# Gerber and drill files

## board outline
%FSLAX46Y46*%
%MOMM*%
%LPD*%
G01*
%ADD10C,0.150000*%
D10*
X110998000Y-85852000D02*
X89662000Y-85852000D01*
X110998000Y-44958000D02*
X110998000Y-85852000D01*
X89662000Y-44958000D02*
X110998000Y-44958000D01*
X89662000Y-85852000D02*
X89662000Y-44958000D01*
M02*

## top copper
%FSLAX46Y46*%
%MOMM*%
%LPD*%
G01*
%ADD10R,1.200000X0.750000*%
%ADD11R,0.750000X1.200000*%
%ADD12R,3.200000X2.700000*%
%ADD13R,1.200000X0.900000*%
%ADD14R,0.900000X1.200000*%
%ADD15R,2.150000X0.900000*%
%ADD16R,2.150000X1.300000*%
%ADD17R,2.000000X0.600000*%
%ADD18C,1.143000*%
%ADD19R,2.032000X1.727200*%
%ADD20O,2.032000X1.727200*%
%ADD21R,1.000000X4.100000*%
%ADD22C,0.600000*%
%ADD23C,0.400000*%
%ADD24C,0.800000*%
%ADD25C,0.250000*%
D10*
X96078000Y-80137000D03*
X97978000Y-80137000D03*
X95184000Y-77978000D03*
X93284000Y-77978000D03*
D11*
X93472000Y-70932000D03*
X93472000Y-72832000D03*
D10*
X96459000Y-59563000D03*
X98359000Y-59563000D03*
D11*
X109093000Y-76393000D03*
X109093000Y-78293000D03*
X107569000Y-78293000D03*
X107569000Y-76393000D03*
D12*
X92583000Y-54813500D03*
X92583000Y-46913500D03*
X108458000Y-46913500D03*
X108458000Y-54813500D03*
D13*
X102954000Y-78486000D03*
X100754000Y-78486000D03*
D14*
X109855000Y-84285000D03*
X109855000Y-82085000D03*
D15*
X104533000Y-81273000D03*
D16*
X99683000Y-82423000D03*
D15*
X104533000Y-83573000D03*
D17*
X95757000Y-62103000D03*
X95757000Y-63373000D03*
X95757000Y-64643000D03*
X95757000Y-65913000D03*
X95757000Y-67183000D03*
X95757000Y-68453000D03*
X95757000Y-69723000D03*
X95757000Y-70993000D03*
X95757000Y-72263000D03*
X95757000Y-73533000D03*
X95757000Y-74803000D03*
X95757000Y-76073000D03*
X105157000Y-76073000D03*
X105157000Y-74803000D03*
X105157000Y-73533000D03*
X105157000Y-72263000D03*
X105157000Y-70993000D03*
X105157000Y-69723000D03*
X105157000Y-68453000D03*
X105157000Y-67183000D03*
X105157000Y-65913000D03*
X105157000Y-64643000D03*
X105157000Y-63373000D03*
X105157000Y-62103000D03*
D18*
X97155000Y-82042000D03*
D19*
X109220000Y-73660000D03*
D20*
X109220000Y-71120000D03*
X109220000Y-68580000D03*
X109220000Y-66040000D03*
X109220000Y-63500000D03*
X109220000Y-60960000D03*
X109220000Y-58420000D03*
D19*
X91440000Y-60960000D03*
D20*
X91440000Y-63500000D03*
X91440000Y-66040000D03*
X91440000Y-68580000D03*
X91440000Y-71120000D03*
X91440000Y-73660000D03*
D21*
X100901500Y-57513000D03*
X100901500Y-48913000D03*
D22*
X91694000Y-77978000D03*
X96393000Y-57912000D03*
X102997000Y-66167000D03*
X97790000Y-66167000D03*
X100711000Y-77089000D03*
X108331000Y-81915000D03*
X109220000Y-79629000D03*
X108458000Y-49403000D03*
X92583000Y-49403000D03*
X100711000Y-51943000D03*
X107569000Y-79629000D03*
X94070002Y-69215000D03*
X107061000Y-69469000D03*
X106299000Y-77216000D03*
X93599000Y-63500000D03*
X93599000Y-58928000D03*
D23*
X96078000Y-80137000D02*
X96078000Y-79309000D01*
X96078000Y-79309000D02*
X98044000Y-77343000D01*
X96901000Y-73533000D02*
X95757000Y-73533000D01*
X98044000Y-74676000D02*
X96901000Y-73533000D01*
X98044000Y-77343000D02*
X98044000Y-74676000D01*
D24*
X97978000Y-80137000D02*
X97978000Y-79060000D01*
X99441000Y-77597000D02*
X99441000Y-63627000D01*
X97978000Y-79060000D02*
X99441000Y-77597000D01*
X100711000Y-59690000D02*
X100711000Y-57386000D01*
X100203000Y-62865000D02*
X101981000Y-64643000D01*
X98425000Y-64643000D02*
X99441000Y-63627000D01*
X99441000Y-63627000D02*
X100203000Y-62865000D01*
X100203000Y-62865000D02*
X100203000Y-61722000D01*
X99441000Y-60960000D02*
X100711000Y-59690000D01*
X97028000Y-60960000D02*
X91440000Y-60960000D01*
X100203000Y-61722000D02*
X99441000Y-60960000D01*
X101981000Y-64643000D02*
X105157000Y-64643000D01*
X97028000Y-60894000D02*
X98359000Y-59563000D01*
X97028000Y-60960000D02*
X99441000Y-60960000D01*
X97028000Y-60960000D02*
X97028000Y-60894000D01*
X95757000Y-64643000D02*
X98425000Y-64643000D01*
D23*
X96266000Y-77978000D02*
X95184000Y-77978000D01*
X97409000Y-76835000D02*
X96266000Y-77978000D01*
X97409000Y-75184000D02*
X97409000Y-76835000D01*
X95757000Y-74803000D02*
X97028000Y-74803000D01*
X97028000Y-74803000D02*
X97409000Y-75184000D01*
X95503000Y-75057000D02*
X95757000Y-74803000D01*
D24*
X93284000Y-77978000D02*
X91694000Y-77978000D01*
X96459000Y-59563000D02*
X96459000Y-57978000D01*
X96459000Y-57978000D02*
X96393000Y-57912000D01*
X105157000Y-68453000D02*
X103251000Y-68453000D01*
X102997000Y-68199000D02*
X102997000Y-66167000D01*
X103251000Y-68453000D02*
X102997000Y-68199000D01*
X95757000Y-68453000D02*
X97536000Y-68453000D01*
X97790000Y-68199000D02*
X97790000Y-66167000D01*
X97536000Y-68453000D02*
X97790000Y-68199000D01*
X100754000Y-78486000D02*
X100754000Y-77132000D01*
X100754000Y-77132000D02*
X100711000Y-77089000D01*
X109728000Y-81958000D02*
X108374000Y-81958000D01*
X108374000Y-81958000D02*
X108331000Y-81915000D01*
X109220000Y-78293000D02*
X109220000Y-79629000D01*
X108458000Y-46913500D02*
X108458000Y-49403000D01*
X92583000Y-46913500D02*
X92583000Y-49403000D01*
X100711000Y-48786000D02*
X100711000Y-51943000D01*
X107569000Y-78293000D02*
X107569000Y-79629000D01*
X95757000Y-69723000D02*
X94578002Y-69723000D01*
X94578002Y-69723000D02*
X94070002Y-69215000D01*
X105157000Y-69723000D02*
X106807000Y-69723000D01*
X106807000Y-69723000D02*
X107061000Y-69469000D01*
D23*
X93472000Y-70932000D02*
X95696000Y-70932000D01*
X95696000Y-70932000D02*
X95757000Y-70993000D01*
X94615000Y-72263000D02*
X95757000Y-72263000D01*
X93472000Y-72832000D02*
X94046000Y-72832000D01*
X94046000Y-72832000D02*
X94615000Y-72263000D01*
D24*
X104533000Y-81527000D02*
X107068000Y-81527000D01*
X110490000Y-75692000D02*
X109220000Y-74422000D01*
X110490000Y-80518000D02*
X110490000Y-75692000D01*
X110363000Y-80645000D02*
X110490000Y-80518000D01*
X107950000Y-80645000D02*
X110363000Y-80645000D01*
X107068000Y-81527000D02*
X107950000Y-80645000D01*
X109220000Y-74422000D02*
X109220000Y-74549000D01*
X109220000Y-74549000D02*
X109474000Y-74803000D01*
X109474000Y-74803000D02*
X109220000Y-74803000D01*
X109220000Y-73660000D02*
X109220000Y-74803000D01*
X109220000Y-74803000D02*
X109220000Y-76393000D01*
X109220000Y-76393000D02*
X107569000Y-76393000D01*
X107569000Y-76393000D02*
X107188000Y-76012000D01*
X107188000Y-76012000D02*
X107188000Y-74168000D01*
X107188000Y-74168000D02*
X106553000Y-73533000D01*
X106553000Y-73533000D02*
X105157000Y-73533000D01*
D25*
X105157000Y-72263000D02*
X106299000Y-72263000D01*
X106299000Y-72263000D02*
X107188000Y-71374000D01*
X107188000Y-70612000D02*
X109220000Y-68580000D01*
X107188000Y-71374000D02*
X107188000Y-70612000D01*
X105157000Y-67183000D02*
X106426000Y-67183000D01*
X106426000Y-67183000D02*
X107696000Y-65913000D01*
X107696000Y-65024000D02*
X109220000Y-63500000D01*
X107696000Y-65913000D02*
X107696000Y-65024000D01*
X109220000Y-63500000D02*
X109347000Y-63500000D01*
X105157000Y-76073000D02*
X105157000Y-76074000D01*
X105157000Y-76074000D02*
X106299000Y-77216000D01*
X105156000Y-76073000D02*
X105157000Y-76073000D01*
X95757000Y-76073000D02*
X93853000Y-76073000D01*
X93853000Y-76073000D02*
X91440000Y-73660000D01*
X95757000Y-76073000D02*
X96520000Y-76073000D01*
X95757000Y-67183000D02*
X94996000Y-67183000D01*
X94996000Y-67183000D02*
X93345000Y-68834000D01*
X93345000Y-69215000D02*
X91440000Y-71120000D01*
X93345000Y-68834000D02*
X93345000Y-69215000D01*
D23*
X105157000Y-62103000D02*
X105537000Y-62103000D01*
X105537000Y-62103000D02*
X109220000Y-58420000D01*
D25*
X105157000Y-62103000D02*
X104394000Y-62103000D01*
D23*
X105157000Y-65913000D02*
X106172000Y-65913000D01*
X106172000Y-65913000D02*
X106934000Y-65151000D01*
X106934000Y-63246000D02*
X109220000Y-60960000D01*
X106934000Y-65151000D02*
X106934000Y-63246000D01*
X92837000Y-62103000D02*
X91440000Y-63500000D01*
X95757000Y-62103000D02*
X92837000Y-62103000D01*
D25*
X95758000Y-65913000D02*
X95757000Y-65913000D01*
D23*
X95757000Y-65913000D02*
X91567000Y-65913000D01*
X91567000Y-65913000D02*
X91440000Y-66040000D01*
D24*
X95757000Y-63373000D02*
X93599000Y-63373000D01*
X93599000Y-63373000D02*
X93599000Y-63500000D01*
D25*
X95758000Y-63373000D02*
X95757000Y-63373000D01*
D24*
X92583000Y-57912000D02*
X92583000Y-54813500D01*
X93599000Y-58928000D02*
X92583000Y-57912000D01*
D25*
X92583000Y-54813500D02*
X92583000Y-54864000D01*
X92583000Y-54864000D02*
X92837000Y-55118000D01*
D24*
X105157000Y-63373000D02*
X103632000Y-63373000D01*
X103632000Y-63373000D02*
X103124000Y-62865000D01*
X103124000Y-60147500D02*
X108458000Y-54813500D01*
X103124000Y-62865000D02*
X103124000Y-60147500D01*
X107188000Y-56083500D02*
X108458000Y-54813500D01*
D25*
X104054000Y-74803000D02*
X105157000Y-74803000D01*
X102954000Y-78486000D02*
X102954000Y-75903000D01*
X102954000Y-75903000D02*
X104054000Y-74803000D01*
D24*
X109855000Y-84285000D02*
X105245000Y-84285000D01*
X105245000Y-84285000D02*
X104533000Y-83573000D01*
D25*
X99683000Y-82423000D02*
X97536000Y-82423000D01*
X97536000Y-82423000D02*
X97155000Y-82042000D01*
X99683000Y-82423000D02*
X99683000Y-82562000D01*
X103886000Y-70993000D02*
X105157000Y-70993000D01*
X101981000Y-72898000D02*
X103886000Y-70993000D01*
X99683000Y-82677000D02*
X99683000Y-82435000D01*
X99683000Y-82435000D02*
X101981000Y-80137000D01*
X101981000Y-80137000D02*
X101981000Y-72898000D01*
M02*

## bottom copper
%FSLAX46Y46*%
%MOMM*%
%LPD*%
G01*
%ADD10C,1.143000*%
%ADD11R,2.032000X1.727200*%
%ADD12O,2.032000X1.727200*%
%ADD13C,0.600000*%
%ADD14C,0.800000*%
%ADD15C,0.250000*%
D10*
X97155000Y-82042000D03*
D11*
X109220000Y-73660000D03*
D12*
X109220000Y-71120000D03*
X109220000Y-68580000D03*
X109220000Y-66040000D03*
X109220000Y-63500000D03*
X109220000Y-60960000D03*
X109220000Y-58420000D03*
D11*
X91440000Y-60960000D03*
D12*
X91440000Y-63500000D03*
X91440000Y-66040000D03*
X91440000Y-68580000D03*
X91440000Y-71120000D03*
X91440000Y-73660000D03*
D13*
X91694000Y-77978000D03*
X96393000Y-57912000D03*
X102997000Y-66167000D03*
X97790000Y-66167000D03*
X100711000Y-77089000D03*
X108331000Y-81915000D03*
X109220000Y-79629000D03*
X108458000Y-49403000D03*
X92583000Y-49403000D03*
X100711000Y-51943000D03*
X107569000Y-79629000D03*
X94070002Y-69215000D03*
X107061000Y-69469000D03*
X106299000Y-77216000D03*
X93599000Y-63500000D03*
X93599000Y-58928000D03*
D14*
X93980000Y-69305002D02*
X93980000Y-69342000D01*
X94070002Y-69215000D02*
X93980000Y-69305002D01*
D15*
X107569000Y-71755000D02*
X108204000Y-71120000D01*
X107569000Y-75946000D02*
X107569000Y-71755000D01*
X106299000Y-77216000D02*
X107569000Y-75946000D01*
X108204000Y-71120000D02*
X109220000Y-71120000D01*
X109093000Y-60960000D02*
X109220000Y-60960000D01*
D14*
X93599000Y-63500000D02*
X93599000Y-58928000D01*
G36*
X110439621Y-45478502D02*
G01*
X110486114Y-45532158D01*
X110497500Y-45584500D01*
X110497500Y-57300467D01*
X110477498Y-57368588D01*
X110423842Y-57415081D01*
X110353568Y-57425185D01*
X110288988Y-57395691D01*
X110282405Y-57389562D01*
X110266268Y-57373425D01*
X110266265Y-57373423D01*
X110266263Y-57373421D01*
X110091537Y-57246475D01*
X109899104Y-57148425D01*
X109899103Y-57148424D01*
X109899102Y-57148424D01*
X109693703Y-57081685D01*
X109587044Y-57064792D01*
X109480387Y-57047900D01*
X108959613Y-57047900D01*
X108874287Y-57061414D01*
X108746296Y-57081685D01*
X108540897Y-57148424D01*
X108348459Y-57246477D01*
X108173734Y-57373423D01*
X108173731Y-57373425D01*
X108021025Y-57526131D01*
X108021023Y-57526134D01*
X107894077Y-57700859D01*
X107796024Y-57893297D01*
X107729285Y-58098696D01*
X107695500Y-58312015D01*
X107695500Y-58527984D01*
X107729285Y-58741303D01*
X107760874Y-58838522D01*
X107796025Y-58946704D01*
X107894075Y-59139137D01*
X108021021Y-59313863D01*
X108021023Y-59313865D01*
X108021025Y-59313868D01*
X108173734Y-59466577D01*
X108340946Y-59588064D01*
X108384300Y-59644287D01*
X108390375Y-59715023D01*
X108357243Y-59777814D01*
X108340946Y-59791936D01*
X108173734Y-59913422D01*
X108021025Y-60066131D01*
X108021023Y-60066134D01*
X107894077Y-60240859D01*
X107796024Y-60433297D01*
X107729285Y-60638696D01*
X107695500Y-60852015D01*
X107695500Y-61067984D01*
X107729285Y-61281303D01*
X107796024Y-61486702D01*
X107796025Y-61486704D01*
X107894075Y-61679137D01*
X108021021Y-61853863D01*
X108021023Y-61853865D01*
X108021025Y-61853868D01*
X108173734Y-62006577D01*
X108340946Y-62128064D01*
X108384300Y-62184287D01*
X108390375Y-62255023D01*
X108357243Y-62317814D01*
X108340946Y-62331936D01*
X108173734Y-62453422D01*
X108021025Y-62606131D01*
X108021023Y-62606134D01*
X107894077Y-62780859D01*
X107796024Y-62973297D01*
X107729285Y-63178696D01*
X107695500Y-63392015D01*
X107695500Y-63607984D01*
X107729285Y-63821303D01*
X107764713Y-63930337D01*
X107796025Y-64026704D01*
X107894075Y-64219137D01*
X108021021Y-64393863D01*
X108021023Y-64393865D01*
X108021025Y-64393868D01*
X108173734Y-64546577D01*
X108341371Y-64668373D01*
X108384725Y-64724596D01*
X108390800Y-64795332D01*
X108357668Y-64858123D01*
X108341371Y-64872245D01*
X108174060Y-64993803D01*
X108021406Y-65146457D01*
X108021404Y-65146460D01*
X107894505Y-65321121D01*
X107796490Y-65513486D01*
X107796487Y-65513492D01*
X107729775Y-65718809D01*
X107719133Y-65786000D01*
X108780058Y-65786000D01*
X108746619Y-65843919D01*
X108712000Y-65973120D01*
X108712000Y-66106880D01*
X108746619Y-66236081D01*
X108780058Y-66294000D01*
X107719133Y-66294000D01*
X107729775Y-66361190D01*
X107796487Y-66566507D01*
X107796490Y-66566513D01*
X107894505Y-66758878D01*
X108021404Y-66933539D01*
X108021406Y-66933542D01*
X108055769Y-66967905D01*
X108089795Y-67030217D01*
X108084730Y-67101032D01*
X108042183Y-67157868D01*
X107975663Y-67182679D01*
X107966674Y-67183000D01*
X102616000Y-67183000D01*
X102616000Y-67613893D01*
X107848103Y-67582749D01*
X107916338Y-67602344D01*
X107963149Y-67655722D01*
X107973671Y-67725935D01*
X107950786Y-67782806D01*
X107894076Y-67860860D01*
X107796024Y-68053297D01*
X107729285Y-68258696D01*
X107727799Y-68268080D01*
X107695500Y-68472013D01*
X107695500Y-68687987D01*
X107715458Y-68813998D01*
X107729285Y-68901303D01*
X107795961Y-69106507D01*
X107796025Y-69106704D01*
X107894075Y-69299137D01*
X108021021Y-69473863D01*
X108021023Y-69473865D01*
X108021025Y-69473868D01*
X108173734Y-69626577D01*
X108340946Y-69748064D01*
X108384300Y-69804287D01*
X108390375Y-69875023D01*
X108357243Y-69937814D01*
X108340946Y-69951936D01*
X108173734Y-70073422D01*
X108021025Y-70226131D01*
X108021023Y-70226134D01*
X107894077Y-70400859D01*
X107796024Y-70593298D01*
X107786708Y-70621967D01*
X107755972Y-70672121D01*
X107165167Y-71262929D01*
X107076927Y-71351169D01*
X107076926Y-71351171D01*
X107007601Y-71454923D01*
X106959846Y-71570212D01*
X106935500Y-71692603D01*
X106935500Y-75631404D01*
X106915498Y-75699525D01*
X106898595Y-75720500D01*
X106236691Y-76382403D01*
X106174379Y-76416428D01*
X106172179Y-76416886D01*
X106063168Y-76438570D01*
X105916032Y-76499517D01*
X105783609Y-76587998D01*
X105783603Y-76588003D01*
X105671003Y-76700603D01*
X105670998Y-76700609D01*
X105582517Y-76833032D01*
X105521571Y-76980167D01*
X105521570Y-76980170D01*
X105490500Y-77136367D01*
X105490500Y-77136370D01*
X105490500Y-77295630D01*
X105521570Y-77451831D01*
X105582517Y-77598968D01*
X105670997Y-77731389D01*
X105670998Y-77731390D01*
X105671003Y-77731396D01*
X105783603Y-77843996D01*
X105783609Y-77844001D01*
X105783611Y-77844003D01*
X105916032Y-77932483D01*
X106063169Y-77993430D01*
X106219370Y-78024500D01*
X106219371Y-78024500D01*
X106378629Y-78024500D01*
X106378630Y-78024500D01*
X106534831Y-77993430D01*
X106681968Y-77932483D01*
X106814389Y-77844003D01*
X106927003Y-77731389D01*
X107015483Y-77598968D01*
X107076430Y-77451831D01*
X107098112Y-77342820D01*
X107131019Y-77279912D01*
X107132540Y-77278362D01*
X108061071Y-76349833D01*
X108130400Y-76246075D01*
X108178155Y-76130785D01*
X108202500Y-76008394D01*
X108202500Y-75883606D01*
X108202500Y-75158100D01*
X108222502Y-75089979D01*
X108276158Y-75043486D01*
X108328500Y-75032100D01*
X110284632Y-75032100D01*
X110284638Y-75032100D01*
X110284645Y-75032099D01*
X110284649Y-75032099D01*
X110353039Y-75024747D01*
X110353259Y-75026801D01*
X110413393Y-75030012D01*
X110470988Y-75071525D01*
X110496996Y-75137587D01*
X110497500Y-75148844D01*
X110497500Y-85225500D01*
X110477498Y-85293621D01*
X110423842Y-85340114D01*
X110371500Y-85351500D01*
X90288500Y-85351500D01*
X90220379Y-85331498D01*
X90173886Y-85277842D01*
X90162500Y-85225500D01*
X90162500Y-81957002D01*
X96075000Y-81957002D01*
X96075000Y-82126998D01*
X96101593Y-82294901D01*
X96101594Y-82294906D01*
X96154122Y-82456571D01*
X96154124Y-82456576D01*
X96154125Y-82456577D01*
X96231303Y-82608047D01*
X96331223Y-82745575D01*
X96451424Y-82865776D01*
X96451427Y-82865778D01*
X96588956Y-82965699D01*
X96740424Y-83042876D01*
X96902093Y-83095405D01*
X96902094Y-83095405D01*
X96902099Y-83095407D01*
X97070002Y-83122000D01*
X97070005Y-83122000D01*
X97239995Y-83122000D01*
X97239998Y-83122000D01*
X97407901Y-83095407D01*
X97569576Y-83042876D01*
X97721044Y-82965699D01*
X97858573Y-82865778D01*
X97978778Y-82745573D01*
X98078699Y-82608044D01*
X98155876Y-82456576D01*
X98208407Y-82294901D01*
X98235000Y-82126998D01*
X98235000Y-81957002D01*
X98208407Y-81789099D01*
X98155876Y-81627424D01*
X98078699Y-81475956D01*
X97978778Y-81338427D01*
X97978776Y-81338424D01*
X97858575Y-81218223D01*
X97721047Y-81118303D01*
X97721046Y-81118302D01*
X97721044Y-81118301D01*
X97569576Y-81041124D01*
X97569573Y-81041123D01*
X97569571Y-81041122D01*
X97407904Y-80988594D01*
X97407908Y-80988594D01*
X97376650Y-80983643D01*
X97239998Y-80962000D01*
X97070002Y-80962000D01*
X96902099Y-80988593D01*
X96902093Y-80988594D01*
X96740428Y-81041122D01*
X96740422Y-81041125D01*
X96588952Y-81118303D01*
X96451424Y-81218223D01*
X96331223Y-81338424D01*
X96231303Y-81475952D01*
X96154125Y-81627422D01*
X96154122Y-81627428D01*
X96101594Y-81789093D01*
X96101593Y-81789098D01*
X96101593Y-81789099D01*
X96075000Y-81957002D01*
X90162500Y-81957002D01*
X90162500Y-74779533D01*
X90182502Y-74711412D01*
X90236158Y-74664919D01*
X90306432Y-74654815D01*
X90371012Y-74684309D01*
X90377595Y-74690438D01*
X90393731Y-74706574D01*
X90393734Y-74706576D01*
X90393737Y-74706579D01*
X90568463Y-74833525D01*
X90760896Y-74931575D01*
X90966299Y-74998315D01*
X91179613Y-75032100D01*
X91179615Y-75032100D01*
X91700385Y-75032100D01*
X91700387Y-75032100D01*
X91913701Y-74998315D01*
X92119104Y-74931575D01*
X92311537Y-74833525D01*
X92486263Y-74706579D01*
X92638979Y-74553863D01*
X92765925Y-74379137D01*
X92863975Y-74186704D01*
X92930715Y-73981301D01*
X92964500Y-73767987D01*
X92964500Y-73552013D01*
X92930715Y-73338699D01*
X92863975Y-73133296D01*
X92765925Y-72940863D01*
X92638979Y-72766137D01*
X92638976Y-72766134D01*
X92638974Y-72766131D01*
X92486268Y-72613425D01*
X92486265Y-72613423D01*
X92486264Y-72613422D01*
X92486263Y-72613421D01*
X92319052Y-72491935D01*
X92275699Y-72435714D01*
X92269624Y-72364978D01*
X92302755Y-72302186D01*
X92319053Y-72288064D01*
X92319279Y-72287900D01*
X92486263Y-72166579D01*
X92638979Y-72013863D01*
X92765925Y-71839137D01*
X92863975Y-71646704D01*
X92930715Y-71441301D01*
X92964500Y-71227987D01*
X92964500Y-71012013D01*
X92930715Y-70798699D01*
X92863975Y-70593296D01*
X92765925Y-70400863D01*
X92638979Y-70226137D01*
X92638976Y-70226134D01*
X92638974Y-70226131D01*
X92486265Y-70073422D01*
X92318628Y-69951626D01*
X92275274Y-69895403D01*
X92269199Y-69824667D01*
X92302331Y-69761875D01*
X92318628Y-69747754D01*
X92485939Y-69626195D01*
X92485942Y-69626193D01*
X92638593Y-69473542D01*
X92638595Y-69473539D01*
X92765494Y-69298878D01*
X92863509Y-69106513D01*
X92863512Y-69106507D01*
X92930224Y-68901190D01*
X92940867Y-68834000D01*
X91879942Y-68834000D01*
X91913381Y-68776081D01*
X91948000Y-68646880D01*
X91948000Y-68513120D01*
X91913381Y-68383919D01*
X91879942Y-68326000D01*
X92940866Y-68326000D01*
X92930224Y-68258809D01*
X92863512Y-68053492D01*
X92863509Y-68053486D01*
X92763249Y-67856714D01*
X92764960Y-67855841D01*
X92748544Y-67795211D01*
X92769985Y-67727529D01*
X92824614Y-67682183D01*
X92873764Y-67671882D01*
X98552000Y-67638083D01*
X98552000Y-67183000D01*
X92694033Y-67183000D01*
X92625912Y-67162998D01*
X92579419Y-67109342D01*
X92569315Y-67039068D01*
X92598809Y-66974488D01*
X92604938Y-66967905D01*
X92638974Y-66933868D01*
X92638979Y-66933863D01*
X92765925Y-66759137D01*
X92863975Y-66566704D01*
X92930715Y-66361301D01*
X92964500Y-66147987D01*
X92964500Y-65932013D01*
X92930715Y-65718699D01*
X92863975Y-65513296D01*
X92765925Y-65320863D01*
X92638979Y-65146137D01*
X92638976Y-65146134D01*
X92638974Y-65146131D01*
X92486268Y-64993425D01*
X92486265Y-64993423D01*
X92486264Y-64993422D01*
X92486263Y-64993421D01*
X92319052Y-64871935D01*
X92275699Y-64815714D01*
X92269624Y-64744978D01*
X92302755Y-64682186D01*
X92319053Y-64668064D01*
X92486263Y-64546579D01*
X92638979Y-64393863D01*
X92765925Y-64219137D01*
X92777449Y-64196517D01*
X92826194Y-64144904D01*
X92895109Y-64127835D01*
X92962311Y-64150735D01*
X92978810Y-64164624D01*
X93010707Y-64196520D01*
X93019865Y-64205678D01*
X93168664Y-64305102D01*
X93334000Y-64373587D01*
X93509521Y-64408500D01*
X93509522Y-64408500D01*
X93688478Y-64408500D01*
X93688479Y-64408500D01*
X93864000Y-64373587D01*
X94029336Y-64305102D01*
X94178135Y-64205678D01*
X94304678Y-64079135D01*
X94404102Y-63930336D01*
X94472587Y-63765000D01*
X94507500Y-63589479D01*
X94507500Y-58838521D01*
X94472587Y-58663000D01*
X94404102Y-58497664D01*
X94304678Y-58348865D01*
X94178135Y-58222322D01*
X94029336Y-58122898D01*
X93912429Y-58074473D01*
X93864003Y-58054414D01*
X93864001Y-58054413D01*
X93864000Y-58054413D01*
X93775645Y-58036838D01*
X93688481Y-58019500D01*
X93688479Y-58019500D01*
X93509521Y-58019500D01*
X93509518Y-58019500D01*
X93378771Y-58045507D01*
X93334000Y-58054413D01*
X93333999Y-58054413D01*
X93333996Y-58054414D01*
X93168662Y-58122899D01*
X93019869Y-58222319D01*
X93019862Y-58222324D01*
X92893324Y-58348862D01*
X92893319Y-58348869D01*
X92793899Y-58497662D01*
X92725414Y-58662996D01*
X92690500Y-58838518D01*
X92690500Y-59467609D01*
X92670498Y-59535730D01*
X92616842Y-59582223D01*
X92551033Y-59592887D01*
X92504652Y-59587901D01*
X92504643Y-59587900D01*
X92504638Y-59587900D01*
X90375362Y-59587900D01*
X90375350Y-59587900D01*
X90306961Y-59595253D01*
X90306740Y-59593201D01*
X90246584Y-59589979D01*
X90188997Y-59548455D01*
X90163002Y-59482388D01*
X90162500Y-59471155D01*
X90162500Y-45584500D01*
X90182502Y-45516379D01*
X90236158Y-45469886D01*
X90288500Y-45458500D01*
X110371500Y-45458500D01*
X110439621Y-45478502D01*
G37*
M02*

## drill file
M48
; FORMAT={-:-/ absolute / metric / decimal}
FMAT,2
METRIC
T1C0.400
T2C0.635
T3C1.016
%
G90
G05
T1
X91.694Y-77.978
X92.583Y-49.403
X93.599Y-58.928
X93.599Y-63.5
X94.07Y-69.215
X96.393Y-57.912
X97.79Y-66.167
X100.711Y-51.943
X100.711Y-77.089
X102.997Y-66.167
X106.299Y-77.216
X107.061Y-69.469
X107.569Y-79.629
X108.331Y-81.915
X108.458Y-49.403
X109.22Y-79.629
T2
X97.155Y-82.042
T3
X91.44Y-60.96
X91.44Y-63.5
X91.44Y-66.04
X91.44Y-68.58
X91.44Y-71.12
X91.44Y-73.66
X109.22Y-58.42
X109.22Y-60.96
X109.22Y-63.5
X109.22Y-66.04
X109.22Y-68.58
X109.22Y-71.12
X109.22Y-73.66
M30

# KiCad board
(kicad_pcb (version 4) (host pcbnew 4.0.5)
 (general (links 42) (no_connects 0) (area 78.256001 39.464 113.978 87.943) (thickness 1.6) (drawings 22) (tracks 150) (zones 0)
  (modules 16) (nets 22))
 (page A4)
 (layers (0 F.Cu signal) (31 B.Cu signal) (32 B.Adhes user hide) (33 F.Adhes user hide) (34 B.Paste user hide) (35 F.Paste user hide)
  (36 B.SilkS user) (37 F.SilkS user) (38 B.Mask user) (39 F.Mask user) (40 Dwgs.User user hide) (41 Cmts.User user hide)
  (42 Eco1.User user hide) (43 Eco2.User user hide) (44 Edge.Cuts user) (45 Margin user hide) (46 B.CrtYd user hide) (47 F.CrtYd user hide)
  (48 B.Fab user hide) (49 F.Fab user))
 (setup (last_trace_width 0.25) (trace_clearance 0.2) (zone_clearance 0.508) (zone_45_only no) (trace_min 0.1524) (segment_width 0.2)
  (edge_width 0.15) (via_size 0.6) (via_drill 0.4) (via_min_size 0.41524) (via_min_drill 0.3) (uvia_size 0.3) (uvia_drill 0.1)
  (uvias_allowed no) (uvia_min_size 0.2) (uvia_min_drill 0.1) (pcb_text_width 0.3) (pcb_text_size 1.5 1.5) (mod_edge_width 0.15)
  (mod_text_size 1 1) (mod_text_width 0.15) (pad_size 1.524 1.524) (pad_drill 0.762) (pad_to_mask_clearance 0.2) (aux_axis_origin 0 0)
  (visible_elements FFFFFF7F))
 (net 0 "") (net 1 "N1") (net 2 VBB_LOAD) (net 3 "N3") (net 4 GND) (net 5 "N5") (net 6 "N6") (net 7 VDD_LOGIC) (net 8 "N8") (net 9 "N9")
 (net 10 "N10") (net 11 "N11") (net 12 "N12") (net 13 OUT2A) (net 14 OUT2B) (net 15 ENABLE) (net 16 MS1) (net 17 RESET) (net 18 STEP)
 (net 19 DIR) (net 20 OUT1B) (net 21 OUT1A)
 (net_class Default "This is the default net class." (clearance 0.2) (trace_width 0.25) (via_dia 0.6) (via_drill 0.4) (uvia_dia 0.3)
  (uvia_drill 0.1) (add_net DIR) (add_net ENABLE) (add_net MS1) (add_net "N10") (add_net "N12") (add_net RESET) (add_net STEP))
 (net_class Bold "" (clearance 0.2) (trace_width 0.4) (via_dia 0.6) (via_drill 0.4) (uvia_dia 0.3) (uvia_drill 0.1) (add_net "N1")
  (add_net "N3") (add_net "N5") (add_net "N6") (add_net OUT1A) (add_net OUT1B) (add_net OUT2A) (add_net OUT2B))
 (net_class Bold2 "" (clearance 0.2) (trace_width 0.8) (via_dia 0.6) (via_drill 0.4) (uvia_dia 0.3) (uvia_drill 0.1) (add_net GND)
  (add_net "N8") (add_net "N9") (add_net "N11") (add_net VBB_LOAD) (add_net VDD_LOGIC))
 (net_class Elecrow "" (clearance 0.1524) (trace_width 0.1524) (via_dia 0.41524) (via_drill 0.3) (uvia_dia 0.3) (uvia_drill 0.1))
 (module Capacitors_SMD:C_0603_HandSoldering (layer F.Cu) (at 97.028 80.137)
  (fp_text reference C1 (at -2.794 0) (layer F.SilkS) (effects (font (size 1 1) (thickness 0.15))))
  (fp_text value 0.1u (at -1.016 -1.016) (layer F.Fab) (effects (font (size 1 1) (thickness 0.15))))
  (pad 1 smd rect (at -0.95 0) (size 1.2 0.75) (layers F.Cu F.Paste F.Mask) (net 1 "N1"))
  (pad 2 smd rect (at 0.95 0) (size 1.2 0.75) (layers F.Cu F.Paste F.Mask) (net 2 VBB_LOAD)))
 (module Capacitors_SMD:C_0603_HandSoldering (layer F.Cu) (at 94.234 77.978 180)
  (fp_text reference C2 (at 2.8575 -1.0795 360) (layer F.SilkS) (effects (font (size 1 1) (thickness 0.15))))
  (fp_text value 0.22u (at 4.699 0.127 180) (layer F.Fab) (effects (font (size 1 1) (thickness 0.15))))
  (pad 1 smd rect (at -0.95 0 180) (size 1.2 0.75) (layers F.Cu F.Paste F.Mask) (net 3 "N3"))
  (pad 2 smd rect (at 0.95 0 180) (size 1.2 0.75) (layers F.Cu F.Paste F.Mask) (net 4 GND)))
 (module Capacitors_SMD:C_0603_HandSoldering (layer F.Cu) (at 93.472 71.882 270)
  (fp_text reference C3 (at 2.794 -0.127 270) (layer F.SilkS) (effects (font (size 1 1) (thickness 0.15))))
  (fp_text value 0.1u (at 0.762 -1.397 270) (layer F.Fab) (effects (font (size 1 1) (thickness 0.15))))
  (pad 1 smd rect (at -0.95 0 270) (size 1.2 0.75) (layers F.Cu F.Paste F.Mask) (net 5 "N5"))
  (pad 2 smd rect (at 0.95 0 270) (size 1.2 0.75) (layers F.Cu F.Paste F.Mask) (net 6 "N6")))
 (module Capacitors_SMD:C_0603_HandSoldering (layer F.Cu) (at 97.409 59.563)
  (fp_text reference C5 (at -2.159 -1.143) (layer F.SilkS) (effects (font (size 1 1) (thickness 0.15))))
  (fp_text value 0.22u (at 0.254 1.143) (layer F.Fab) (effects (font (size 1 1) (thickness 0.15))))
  (pad 1 smd rect (at -0.95 0) (size 1.2 0.75) (layers F.Cu F.Paste F.Mask) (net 4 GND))
  (pad 2 smd rect (at 0.95 0) (size 1.2 0.75) (layers F.Cu F.Paste F.Mask) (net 2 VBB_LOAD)))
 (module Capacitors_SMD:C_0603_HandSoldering (layer F.Cu) (at 109.093 77.343 270)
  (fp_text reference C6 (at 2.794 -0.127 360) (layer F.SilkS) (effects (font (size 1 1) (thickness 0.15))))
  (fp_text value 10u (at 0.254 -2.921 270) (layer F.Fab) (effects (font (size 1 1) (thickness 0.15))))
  (pad 1 smd rect (at -0.95 0 270) (size 1.2 0.75) (layers F.Cu F.Paste F.Mask) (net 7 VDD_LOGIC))
  (pad 2 smd rect (at 0.95 0 270) (size 1.2 0.75) (layers F.Cu F.Paste F.Mask) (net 4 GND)))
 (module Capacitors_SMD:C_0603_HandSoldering (layer F.Cu) (at 107.569 77.343 90)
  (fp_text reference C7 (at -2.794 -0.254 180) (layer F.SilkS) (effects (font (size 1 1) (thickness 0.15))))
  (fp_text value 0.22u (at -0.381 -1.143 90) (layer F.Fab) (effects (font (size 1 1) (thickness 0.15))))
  (pad 1 smd rect (at -0.95 0 90) (size 1.2 0.75) (layers F.Cu F.Paste F.Mask) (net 4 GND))
  (pad 2 smd rect (at 0.95 0 90) (size 1.2 0.75) (layers F.Cu F.Paste F.Mask) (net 7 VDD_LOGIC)))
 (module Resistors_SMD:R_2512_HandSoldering (layer F.Cu) (at 92.583 50.8635 90)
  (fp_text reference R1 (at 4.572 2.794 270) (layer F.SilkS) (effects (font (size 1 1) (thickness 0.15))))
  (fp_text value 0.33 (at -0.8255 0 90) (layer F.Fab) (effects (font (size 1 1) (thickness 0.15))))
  (pad 1 smd rect (at -3.95 0 90) (size 2.7 3.2) (layers F.Cu F.Paste F.Mask) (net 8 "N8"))
  (pad 2 smd rect (at 3.95 0 90) (size 2.7 3.2) (layers F.Cu F.Paste F.Mask) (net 4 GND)))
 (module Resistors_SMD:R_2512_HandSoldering (layer F.Cu) (at 108.458 50.8635 270)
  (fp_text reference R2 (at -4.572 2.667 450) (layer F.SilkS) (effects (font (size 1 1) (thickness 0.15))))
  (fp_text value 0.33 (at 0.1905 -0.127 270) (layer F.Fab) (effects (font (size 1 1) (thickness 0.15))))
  (pad 1 smd rect (at -3.95 0 270) (size 2.7 3.2) (layers F.Cu F.Paste F.Mask) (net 4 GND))
  (pad 2 smd rect (at 3.95 0 270) (size 2.7 3.2) (layers F.Cu F.Paste F.Mask) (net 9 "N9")))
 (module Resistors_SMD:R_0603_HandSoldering (layer F.Cu) (at 101.854 78.486 180)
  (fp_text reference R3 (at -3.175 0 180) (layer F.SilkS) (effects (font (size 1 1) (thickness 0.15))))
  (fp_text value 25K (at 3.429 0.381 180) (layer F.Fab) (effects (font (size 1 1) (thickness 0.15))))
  (pad 1 smd rect (at -1.1 0 180) (size 1.2 0.9) (layers F.Cu F.Paste F.Mask) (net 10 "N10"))
  (pad 2 smd rect (at 1.1 0 180) (size 1.2 0.9) (layers F.Cu F.Paste F.Mask) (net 4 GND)))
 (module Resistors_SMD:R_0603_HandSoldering (layer F.Cu) (at 109.855 83.185 90)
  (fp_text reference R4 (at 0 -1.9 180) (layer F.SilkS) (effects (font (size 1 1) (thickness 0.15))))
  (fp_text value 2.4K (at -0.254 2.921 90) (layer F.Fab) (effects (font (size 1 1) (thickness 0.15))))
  (pad 1 smd rect (at -1.1 0 90) (size 1.2 0.9) (layers F.Cu F.Paste F.Mask) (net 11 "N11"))
  (pad 2 smd rect (at 1.1 0 90) (size 1.2 0.9) (layers F.Cu F.Paste F.Mask) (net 4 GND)))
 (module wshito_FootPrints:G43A (layer F.Cu) (at 102.108 82.423 90)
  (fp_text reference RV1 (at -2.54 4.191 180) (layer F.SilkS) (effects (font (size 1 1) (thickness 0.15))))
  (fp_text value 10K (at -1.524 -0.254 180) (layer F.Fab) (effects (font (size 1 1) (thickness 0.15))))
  (pad 1 smd rect (at 1.15 2.425 90) (size 0.9 2.15) (layers F.Cu F.Paste F.Mask) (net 7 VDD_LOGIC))
  (pad 2 smd rect (at 0 -2.425 90) (size 1.3 2.15) (layers F.Cu F.Paste F.Mask) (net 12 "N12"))
  (pad 3 smd rect (at -1.15 2.425 90) (size 0.9 2.15) (layers F.Cu F.Paste F.Mask) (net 11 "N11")))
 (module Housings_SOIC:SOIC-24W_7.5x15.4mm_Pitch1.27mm (layer F.Cu) (at 100.457 69.088)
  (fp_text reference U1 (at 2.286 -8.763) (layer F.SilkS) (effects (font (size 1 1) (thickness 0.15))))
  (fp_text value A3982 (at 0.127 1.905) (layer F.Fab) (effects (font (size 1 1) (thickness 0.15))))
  (pad 1 smd rect (at -4.7 -6.985) (size 2 0.6) (layers F.Cu F.Paste F.Mask) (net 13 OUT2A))
  (pad 2 smd rect (at -4.7 -5.715) (size 2 0.6) (layers F.Cu F.Paste F.Mask) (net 8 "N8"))
  (pad 3 smd rect (at -4.7 -4.445) (size 2 0.6) (layers F.Cu F.Paste F.Mask) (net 2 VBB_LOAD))
  (pad 4 smd rect (at -4.7 -3.175) (size 2 0.6) (layers F.Cu F.Paste F.Mask) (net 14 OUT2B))
  (pad 5 smd rect (at -4.7 -1.905) (size 2 0.6) (layers F.Cu F.Paste F.Mask) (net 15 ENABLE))
  (pad 6 smd rect (at -4.7 -0.635) (size 2 0.6) (layers F.Cu F.Paste F.Mask) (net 4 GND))
  (pad 7 smd rect (at -4.7 0.635) (size 2 0.6) (layers F.Cu F.Paste F.Mask) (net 4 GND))
  (pad 8 smd rect (at -4.7 1.905) (size 2 0.6) (layers F.Cu F.Paste F.Mask) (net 5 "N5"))
  (pad 9 smd rect (at -4.7 3.175) (size 2 0.6) (layers F.Cu F.Paste F.Mask) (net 6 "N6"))
  (pad 10 smd rect (at -4.7 4.445) (size 2 0.6) (layers F.Cu F.Paste F.Mask) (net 1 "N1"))
  (pad 11 smd rect (at -4.7 5.715) (size 2 0.6) (layers F.Cu F.Paste F.Mask) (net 3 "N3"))
  (pad 12 smd rect (at -4.7 6.985) (size 2 0.6) (layers F.Cu F.Paste F.Mask) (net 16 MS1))
  (pad 13 smd rect (at 4.7 6.985) (size 2 0.6) (layers F.Cu F.Paste F.Mask) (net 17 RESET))
  (pad 14 smd rect (at 4.7 5.715) (size 2 0.6) (layers F.Cu F.Paste F.Mask) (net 10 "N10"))
  (pad 15 smd rect (at 4.7 4.445) (size 2 0.6) (layers F.Cu F.Paste F.Mask) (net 7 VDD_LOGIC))
  (pad 16 smd rect (at 4.7 3.175) (size 2 0.6) (layers F.Cu F.Paste F.Mask) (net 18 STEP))
  (pad 17 smd rect (at 4.7 1.905) (size 2 0.6) (layers F.Cu F.Paste F.Mask) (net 12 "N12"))
  (pad 18 smd rect (at 4.7 0.635) (size 2 0.6) (layers F.Cu F.Paste F.Mask) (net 4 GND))
  (pad 19 smd rect (at 4.7 -0.635) (size 2 0.6) (layers F.Cu F.Paste F.Mask) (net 4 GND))
  (pad 20 smd rect (at 4.7 -1.905) (size 2 0.6) (layers F.Cu F.Paste F.Mask) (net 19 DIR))
  (pad 21 smd rect (at 4.7 -3.175) (size 2 0.6) (layers F.Cu F.Paste F.Mask) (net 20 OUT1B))
  (pad 22 smd rect (at 4.7 -4.445) (size 2 0.6) (layers F.Cu F.Paste F.Mask) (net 2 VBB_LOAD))
  (pad 23 smd rect (at 4.7 -5.715) (size 2 0.6) (layers F.Cu F.Paste F.Mask) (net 9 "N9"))
  (pad 24 smd rect (at 4.7 -6.985) (size 2 0.6) (layers F.Cu F.Paste F.Mask) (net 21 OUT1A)))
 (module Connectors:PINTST (layer F.Cu) (at 97.155 82.042)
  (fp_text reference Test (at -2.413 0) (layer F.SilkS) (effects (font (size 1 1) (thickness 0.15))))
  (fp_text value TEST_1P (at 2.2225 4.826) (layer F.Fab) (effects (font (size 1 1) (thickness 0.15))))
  (pad 1 thru_hole circle (at 0 0) (size 1.143 1.143) (drill 0.635) (layers *.Cu *.Mask) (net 12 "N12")))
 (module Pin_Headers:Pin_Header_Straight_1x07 (layer F.Cu) (at 109.22 73.66 180)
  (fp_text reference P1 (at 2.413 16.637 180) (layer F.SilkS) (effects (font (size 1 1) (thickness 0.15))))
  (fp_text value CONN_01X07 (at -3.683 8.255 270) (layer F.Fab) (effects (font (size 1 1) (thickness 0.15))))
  (pad 1 thru_hole rect (at 0 0 180) (size 2.032 1.7272) (drill 1.016) (layers *.Cu *.Mask) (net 7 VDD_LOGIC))
  (pad 2 thru_hole oval (at 0 2.54 180) (size 2.032 1.7272) (drill 1.016) (layers *.Cu *.Mask) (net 17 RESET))
  (pad 3 thru_hole oval (at 0 5.08 180) (size 2.032 1.7272) (drill 1.016) (layers *.Cu *.Mask) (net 18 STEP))
  (pad 4 thru_hole oval (at 0 7.62 180) (size 2.032 1.7272) (drill 1.016) (layers *.Cu *.Mask) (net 4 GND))
  (pad 5 thru_hole oval (at 0 10.16 180) (size 2.032 1.7272) (drill 1.016) (layers *.Cu *.Mask) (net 19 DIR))
  (pad 6 thru_hole oval (at 0 12.7 180) (size 2.032 1.7272) (drill 1.016) (layers *.Cu *.Mask) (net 20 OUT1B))
  (pad 7 thru_hole oval (at 0 15.24 180) (size 2.032 1.7272) (drill 1.016) (layers *.Cu *.Mask) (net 21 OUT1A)))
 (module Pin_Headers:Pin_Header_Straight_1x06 (layer F.Cu) (at 91.44 60.96)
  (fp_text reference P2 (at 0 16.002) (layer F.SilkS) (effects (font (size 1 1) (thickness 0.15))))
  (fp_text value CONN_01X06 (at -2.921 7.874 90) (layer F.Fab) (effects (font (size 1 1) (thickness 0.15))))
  (pad 1 thru_hole rect (at 0 0) (size 2.032 1.7272) (drill 1.016) (layers *.Cu *.Mask) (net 2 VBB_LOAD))
  (pad 2 thru_hole oval (at 0 2.54) (size 2.032 1.7272) (drill 1.016) (layers *.Cu *.Mask) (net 13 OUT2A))
  (pad 3 thru_hole oval (at 0 5.08) (size 2.032 1.7272) (drill 1.016) (layers *.Cu *.Mask) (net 14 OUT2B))
  (pad 4 thru_hole oval (at 0 7.62) (size 2.032 1.7272) (drill 1.016) (layers *.Cu *.Mask) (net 4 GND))
  (pad 5 thru_hole oval (at 0 10.16) (size 2.032 1.7272) (drill 1.016) (layers *.Cu *.Mask) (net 15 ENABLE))
  (pad 6 thru_hole oval (at 0 12.7) (size 2.032 1.7272) (drill 1.016) (layers *.Cu *.Mask) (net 16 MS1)))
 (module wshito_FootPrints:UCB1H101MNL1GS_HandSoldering (layer F.Cu) (at 100.9015 53.213 180)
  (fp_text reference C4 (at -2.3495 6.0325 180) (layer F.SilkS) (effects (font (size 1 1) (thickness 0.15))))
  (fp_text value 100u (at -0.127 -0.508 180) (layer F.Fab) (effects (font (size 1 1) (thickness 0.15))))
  (pad 1 smd rect (at 0 -4.3 180) (size 1 4.1) (layers F.Cu F.Paste F.Mask) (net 2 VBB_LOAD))
  (pad 2 smd rect (at 0 4.3 180) (size 1 4.1) (layers F.Cu F.Paste F.Mask) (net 4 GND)))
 (gr_line (start 110.998 85.852) (end 89.662 85.852) (angle 90) (layer Edge.Cuts) (width 0.15))
 (gr_line (start 110.998 44.958) (end 110.998 85.852) (angle 90) (layer Edge.Cuts) (width 0.15))
 (gr_line (start 89.662 44.958) (end 110.998 44.958) (angle 90) (layer Edge.Cuts) (width 0.15))
 (gr_line (start 89.662 85.852) (end 89.662 44.958) (angle 90) (layer Edge.Cuts) (width 0.15))
 (segment (start 96.078 80.137) (end 96.078 79.309) (width 0.4) (layer F.Cu) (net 1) (status 10))
 (segment (start 96.078 79.309) (end 98.044 77.343) (width 0.4) (layer F.Cu) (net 1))
 (segment (start 96.901 73.533) (end 95.757 73.533) (width 0.4) (layer F.Cu) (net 1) (status 20))
 (segment (start 98.044 74.676) (end 96.901 73.533) (width 0.4) (layer F.Cu) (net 1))
 (segment (start 98.044 77.343) (end 98.044 74.676) (width 0.4) (layer F.Cu) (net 1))
 (segment (start 97.978 80.137) (end 97.978 79.06) (width 0.8) (layer F.Cu) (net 2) (status 10))
 (segment (start 99.441 77.597) (end 99.441 63.627) (width 0.8) (layer F.Cu) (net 2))
 (segment (start 97.978 79.06) (end 99.441 77.597) (width 0.8) (layer F.Cu) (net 2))
 (segment (start 100.711 59.69) (end 100.711 57.386) (width 0.8) (layer F.Cu) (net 2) (status 20))
 (segment (start 100.203 62.865) (end 101.981 64.643) (width 0.8) (layer F.Cu) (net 2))
 (segment (start 98.425 64.643) (end 99.441 63.627) (width 0.8) (layer F.Cu) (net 2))
 (segment (start 99.441 63.627) (end 100.203 62.865) (width 0.8) (layer F.Cu) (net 2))
 (segment (start 100.203 62.865) (end 100.203 61.722) (width 0.8) (layer F.Cu) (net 2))
 (segment (start 99.441 60.96) (end 100.711 59.69) (width 0.8) (layer F.Cu) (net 2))
 (segment (start 97.028 60.96) (end 91.44 60.96) (width 0.8) (layer F.Cu) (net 2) (status 20))
 (segment (start 100.203 61.722) (end 99.441 60.96) (width 0.8) (layer F.Cu) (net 2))
 (segment (start 101.981 64.643) (end 105.157 64.643) (width 0.8) (layer F.Cu) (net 2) (status 20))
 (segment (start 97.028 60.894) (end 98.359 59.563) (width 0.8) (layer F.Cu) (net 2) (status 20))
 (segment (start 97.028 60.96) (end 99.441 60.96) (width 0.8) (layer F.Cu) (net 2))
 (segment (start 97.028 60.96) (end 97.028 60.894) (width 0.8) (layer F.Cu) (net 2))
 (segment (start 95.757 64.643) (end 98.425 64.643) (width 0.8) (layer F.Cu) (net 2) (status 10))
 (segment (start 96.266 77.978) (end 95.184 77.978) (width 0.4) (layer F.Cu) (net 3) (status 20))
 (segment (start 97.409 76.835) (end 96.266 77.978) (width 0.4) (layer F.Cu) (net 3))
 (segment (start 97.409 75.184) (end 97.409 76.835) (width 0.4) (layer F.Cu) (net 3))
 (segment (start 95.757 74.803) (end 97.028 74.803) (width 0.4) (layer F.Cu) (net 3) (status 10))
 (segment (start 97.028 74.803) (end 97.409 75.184) (width 0.4) (layer F.Cu) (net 3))
 (segment (start 95.503 75.057) (end 95.757 74.803) (width 0.4) (layer F.Cu) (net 3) (status 30))
 (segment (start 93.284 77.978) (end 91.694 77.978) (width 0.8) (layer F.Cu) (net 4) (status 10))
 (via (at 91.694 77.978) (size 0.6) (drill 0.4) (layers F.Cu B.Cu) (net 4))
 (segment (start 96.459 59.563) (end 96.459 57.978) (width 0.8) (layer F.Cu) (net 4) (status 10))
 (via (at 96.393 57.912) (size 0.6) (drill 0.4) (layers F.Cu B.Cu) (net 4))
 (segment (start 96.459 57.978) (end 96.393 57.912) (width 0.8) (layer F.Cu) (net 4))
 (segment (start 105.157 68.453) (end 103.251 68.453) (width 0.8) (layer F.Cu) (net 4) (status 10))
 (via (at 102.997 66.167) (size 0.6) (drill 0.4) (layers F.Cu B.Cu) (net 4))
 (segment (start 102.997 68.199) (end 102.997 66.167) (width 0.8) (layer F.Cu) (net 4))
 (segment (start 103.251 68.453) (end 102.997 68.199) (width 0.8) (layer F.Cu) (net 4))
 (segment (start 95.757 68.453) (end 97.536 68.453) (width 0.8) (layer F.Cu) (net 4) (status 10))
 (via (at 97.79 66.167) (size 0.6) (drill 0.4) (layers F.Cu B.Cu) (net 4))
 (segment (start 97.79 68.199) (end 97.79 66.167) (width 0.8) (layer F.Cu) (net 4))
 (segment (start 97.536 68.453) (end 97.79 68.199) (width 0.8) (layer F.Cu) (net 4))
 (segment (start 100.754 78.486) (end 100.754 77.132) (width 0.8) (layer F.Cu) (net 4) (status 10))
 (via (at 100.711 77.089) (size 0.6) (drill 0.4) (layers F.Cu B.Cu) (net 4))
 (segment (start 100.754 77.132) (end 100.711 77.089) (width 0.8) (layer F.Cu) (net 4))
 (segment (start 109.728 81.958) (end 108.374 81.958) (width 0.8) (layer F.Cu) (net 4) (status 10))
 (via (at 108.331 81.915) (size 0.6) (drill 0.4) (layers F.Cu B.Cu) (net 4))
 (segment (start 108.374 81.958) (end 108.331 81.915) (width 0.8) (layer F.Cu) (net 4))
 (segment (start 109.22 78.293) (end 109.22 79.629) (width 0.8) (layer F.Cu) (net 4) (status 10))
 (via (at 109.22 79.629) (size 0.6) (drill 0.4) (layers F.Cu B.Cu) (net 4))
 (segment (start 108.458 46.9135) (end 108.458 49.403) (width 0.8) (layer F.Cu) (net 4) (status 10))
 (via (at 108.458 49.403) (size 0.6) (drill 0.4) (layers F.Cu B.Cu) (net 4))
 (segment (start 92.583 46.9135) (end 92.583 49.403) (width 0.8) (layer F.Cu) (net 4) (status 10))
 (via (at 92.583 49.403) (size 0.6) (drill 0.4) (layers F.Cu B.Cu) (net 4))
 (segment (start 100.711 48.786) (end 100.711 51.943) (width 0.8) (layer F.Cu) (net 4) (status 10))
 (via (at 100.711 51.943) (size 0.6) (drill 0.4) (layers F.Cu B.Cu) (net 4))
 (segment (start 107.569 78.293) (end 107.569 79.629) (width 0.8) (layer F.Cu) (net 4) (status 10))
 (via (at 107.569 79.629) (size 0.6) (drill 0.4) (layers F.Cu B.Cu) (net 4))
 (segment (start 95.757 69.723) (end 94.578002 69.723) (width 0.8) (layer F.Cu) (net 4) (status 10))
 (segment (start 93.98 69.305002) (end 93.98 69.342) (width 0.8) (layer B.Cu) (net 4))
 (segment (start 94.070002 69.215) (end 93.98 69.305002) (width 0.8) (layer B.Cu) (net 4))
 (via (at 94.070002 69.215) (size 0.6) (drill 0.4) (layers F.Cu B.Cu) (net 4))
 (segment (start 94.578002 69.723) (end 94.070002 69.215) (width 0.8) (layer F.Cu) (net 4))
 (segment (start 105.157 69.723) (end 106.807 69.723) (width 0.8) (layer F.Cu) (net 4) (status 10))
 (via (at 107.061 69.469) (size 0.6) (drill 0.4) (layers F.Cu B.Cu) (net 4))
 (segment (start 106.807 69.723) (end 107.061 69.469) (width 0.8) (layer F.Cu) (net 4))
 (segment (start 93.472 70.932) (end 95.696 70.932) (width 0.4) (layer F.Cu) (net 5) (status 30))
 (segment (start 95.696 70.932) (end 95.757 70.993) (width 0.4) (layer F.Cu) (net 5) (status 30))
 (segment (start 94.615 72.263) (end 95.757 72.263) (width 0.4) (layer F.Cu) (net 6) (status 20))
 (segment (start 93.472 72.832) (end 94.046 72.832) (width 0.4) (layer F.Cu) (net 6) (status 10))
 (segment (start 94.046 72.832) (end 94.615 72.263) (width 0.4) (layer F.Cu) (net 6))
 (segment (start 104.533 81.527) (end 107.068 81.527) (width 0.8) (layer F.Cu) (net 7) (status 10))
 (segment (start 110.49 75.692) (end 109.22 74.422) (width 0.8) (layer F.Cu) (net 7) (status 20))
 (segment (start 110.49 80.518) (end 110.49 75.692) (width 0.8) (layer F.Cu) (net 7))
 (segment (start 110.363 80.645) (end 110.49 80.518) (width 0.8) (layer F.Cu) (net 7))
 (segment (start 107.95 80.645) (end 110.363 80.645) (width 0.8) (layer F.Cu) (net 7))
 (segment (start 107.068 81.527) (end 107.95 80.645) (width 0.8) (layer F.Cu) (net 7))
 (segment (start 109.22 74.422) (end 109.22 74.549) (width 0.8) (layer F.Cu) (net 7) (status 10))
 (segment (start 109.22 74.549) (end 109.474 74.803) (width 0.8) (layer F.Cu) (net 7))
 (segment (start 109.474 74.803) (end 109.22 74.803) (width 0.8) (layer F.Cu) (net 7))
 (segment (start 109.22 73.66) (end 109.22 74.803) (width 0.8) (layer F.Cu) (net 7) (status 10))
 (segment (start 109.22 74.803) (end 109.22 76.393) (width 0.8) (layer F.Cu) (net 7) (status 20))
 (segment (start 109.22 76.393) (end 107.569 76.393) (width 0.8) (layer F.Cu) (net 7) (status 30))
 (segment (start 107.569 76.393) (end 107.188 76.012) (width 0.8) (layer F.Cu) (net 7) (status 10))
 (segment (start 107.188 76.012) (end 107.188 74.168) (width 0.8) (layer F.Cu) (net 7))
 (segment (start 107.188 74.168) (end 106.553 73.533) (width 0.8) (layer F.Cu) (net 7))
 (segment (start 106.553 73.533) (end 105.157 73.533) (width 0.8) (layer F.Cu) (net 7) (status 20))
 (segment (start 105.157 72.263) (end 106.299 72.263) (width 0.25) (layer F.Cu) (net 18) (status 10))
 (segment (start 106.299 72.263) (end 107.188 71.374) (width 0.25) (layer F.Cu) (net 18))
 (segment (start 107.188 70.612) (end 109.22 68.58) (width 0.25) (layer F.Cu) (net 18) (status 20))
 (segment (start 107.188 71.374) (end 107.188 70.612) (width 0.25) (layer F.Cu) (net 18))
 (segment (start 105.157 67.183) (end 106.426 67.183) (width 0.25) (layer F.Cu) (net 19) (status 10))
 (segment (start 106.426 67.183) (end 107.696 65.913) (width 0.25) (layer F.Cu) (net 19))
 (segment (start 107.696 65.024) (end 109.22 63.5) (width 0.25) (layer F.Cu) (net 19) (status 20))
 (segment (start 107.696 65.913) (end 107.696 65.024) (width 0.25) (layer F.Cu) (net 19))
 (segment (start 109.22 63.5) (end 109.347 63.5) (width 0.25) (layer F.Cu) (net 19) (status 80030))
 (segment (start 105.157 76.073) (end 105.157 76.074) (width 0.25) (layer F.Cu) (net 17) (status 30))
 (segment (start 105.157 76.074) (end 106.299 77.216) (width 0.25) (layer F.Cu) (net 17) (status 10))
 (segment (start 107.569 71.755) (end 108.204 71.12) (width 0.25) (layer B.Cu) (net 17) (status 20))
 (segment (start 107.569 75.946) (end 107.569 71.755) (width 0.25) (layer B.Cu) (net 17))
 (segment (start 106.299 77.216) (end 107.569 75.946) (width 0.25) (layer B.Cu) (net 17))
 (via (at 106.299 77.216) (size 0.6) (drill 0.4) (layers F.Cu B.Cu) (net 17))
 (segment (start 108.204 71.12) (end 109.22 71.12) (width 0.25) (layer B.Cu) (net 17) (status 30))
 (segment (start 105.156 76.073) (end 105.157 76.073) (width 0.25) (layer F.Cu) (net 17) (status 80030))
 (segment (start 95.757 76.073) (end 93.853 76.073) (width 0.25) (layer F.Cu) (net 16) (status 10))
 (segment (start 93.853 76.073) (end 91.44 73.66) (width 0.25) (layer F.Cu) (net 16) (status 20))
 (segment (start 95.757 76.073) (end 96.52 76.073) (width 0.25) (layer F.Cu) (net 16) (status 80030))
 (segment (start 95.757 67.183) (end 94.996 67.183) (width 0.25) (layer F.Cu) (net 15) (status 30))
 (segment (start 94.996 67.183) (end 93.345 68.834) (width 0.25) (layer F.Cu) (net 15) (status 10))
 (segment (start 93.345 69.215) (end 91.44 71.12) (width 0.25) (layer F.Cu) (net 15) (status 20))
 (segment (start 93.345 68.834) (end 93.345 69.215) (width 0.25) (layer F.Cu) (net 15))
 (segment (start 105.157 62.103) (end 105.537 62.103) (width 0.4) (layer F.Cu) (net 21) (status 30))
 (segment (start 105.537 62.103) (end 109.22 58.42) (width 0.4) (layer F.Cu) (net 21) (status 30))
 (segment (start 105.157 62.103) (end 104.394 62.103) (width 0.25) (layer F.Cu) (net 21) (status 80030))
 (segment (start 105.157 65.913) (end 106.172 65.913) (width 0.4) (layer F.Cu) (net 20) (status 10))
 (segment (start 106.172 65.913) (end 106.934 65.151) (width 0.4) (layer F.Cu) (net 20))
 (segment (start 106.934 63.246) (end 109.22 60.96) (width 0.4) (layer F.Cu) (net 20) (status 20))
 (segment (start 106.934 65.151) (end 106.934 63.246) (width 0.4) (layer F.Cu) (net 20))
 (segment (start 109.093 60.96) (end 109.22 60.96) (width 0.25) (layer B.Cu) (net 20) (status 80030))
 (segment (start 92.837 62.103) (end 91.44 63.5) (width 0.4) (layer F.Cu) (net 13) (status 20))
 (segment (start 95.757 62.103) (end 92.837 62.103) (width 0.4) (layer F.Cu) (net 13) (status 10))
 (segment (start 95.758 65.913) (end 95.757 65.913) (width 0.25) (layer F.Cu) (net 14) (status 80030))
 (segment (start 95.757 65.913) (end 91.567 65.913) (width 0.4) (layer F.Cu) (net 14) (status 30))
 (segment (start 91.567 65.913) (end 91.44 66.04) (width 0.4) (layer F.Cu) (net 14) (status 30))
 (segment (start 95.757 63.373) (end 93.599 63.373) (width 0.8) (layer F.Cu) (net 8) (status 10))
 (via (at 93.599 63.5) (size 0.6) (drill 0.4) (layers F.Cu B.Cu) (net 8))
 (segment (start 93.599 63.373) (end 93.599 63.5) (width 0.8) (layer F.Cu) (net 8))
 (segment (start 95.758 63.373) (end 95.757 63.373) (width 0.25) (layer F.Cu) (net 8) (status 80030))
 (segment (start 92.583 57.912) (end 92.583 54.8135) (width 0.8) (layer F.Cu) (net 8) (status 20))
 (segment (start 93.599 58.928) (end 92.583 57.912) (width 0.8) (layer F.Cu) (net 8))
 (via (at 93.599 58.928) (size 0.6) (drill 0.4) (layers F.Cu B.Cu) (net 8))
 (segment (start 93.599 63.5) (end 93.599 58.928) (width 0.8) (layer B.Cu) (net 8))
 (segment (start 92.583 54.8135) (end 92.583 54.864) (width 0.25) (layer F.Cu) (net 8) (status 80030))
 (segment (start 92.583 54.864) (end 92.837 55.118) (width 0.25) (layer F.Cu) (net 8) (status 80030))
 (segment (start 105.157 63.373) (end 103.632 63.373) (width 0.8) (layer F.Cu) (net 9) (status 10))
 (segment (start 103.632 63.373) (end 103.124 62.865) (width 0.8) (layer F.Cu) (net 9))
 (segment (start 103.124 60.1475) (end 108.458 54.8135) (width 0.8) (layer F.Cu) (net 9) (status 20))
 (segment (start 103.124 62.865) (end 103.124 60.1475) (width 0.8) (layer F.Cu) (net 9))
 (segment (start 107.188 56.0835) (end 108.458 54.8135) (width 0.8) (layer F.Cu) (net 9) (status 30))
 (segment (start 104.054 74.803) (end 105.157 74.803) (width 0.25) (layer F.Cu) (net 10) (status 20))
 (segment (start 102.954 78.486) (end 102.954 75.903) (width 0.25) (layer F.Cu) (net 10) (status 10))
 (segment (start 102.954 75.903) (end 104.054 74.803) (width 0.25) (layer F.Cu) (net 10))
 (segment (start 109.855 84.285) (end 105.245 84.285) (width 0.8) (layer F.Cu) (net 11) (status 10))
 (segment (start 105.245 84.285) (end 104.533 83.573) (width 0.8) (layer F.Cu) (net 11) (status 20))
 (segment (start 99.683 82.423) (end 97.536 82.423) (width 0.25) (layer F.Cu) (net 12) (status 30))
 (segment (start 97.536 82.423) (end 97.155 82.042) (width 0.25) (layer F.Cu) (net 12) (status 30))
 (segment (start 99.683 82.423) (end 99.683 82.562) (width 0.25) (layer F.Cu) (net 12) (status 30))
 (segment (start 103.886 70.993) (end 105.157 70.993) (width 0.25) (layer F.Cu) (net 12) (status 20))
 (segment (start 101.981 72.898) (end 103.886 70.993) (width 0.25) (layer F.Cu) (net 12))
 (segment (start 99.683 82.677) (end 99.683 82.435) (width 0.25) (layer F.Cu) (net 12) (status 30))
 (segment (start 99.683 82.435) (end 101.981 80.137) (width 0.25) (layer F.Cu) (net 12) (status 10))
 (segment (start 101.981 80.137) (end 101.981 72.898) (width 0.25) (layer F.Cu) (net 12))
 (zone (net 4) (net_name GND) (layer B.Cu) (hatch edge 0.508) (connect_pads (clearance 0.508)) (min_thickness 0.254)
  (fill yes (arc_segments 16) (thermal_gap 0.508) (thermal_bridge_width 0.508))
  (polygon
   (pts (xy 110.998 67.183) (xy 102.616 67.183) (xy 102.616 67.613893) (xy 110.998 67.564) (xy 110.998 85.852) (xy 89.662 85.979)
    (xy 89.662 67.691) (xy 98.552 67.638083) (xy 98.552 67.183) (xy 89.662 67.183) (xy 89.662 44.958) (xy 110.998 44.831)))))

